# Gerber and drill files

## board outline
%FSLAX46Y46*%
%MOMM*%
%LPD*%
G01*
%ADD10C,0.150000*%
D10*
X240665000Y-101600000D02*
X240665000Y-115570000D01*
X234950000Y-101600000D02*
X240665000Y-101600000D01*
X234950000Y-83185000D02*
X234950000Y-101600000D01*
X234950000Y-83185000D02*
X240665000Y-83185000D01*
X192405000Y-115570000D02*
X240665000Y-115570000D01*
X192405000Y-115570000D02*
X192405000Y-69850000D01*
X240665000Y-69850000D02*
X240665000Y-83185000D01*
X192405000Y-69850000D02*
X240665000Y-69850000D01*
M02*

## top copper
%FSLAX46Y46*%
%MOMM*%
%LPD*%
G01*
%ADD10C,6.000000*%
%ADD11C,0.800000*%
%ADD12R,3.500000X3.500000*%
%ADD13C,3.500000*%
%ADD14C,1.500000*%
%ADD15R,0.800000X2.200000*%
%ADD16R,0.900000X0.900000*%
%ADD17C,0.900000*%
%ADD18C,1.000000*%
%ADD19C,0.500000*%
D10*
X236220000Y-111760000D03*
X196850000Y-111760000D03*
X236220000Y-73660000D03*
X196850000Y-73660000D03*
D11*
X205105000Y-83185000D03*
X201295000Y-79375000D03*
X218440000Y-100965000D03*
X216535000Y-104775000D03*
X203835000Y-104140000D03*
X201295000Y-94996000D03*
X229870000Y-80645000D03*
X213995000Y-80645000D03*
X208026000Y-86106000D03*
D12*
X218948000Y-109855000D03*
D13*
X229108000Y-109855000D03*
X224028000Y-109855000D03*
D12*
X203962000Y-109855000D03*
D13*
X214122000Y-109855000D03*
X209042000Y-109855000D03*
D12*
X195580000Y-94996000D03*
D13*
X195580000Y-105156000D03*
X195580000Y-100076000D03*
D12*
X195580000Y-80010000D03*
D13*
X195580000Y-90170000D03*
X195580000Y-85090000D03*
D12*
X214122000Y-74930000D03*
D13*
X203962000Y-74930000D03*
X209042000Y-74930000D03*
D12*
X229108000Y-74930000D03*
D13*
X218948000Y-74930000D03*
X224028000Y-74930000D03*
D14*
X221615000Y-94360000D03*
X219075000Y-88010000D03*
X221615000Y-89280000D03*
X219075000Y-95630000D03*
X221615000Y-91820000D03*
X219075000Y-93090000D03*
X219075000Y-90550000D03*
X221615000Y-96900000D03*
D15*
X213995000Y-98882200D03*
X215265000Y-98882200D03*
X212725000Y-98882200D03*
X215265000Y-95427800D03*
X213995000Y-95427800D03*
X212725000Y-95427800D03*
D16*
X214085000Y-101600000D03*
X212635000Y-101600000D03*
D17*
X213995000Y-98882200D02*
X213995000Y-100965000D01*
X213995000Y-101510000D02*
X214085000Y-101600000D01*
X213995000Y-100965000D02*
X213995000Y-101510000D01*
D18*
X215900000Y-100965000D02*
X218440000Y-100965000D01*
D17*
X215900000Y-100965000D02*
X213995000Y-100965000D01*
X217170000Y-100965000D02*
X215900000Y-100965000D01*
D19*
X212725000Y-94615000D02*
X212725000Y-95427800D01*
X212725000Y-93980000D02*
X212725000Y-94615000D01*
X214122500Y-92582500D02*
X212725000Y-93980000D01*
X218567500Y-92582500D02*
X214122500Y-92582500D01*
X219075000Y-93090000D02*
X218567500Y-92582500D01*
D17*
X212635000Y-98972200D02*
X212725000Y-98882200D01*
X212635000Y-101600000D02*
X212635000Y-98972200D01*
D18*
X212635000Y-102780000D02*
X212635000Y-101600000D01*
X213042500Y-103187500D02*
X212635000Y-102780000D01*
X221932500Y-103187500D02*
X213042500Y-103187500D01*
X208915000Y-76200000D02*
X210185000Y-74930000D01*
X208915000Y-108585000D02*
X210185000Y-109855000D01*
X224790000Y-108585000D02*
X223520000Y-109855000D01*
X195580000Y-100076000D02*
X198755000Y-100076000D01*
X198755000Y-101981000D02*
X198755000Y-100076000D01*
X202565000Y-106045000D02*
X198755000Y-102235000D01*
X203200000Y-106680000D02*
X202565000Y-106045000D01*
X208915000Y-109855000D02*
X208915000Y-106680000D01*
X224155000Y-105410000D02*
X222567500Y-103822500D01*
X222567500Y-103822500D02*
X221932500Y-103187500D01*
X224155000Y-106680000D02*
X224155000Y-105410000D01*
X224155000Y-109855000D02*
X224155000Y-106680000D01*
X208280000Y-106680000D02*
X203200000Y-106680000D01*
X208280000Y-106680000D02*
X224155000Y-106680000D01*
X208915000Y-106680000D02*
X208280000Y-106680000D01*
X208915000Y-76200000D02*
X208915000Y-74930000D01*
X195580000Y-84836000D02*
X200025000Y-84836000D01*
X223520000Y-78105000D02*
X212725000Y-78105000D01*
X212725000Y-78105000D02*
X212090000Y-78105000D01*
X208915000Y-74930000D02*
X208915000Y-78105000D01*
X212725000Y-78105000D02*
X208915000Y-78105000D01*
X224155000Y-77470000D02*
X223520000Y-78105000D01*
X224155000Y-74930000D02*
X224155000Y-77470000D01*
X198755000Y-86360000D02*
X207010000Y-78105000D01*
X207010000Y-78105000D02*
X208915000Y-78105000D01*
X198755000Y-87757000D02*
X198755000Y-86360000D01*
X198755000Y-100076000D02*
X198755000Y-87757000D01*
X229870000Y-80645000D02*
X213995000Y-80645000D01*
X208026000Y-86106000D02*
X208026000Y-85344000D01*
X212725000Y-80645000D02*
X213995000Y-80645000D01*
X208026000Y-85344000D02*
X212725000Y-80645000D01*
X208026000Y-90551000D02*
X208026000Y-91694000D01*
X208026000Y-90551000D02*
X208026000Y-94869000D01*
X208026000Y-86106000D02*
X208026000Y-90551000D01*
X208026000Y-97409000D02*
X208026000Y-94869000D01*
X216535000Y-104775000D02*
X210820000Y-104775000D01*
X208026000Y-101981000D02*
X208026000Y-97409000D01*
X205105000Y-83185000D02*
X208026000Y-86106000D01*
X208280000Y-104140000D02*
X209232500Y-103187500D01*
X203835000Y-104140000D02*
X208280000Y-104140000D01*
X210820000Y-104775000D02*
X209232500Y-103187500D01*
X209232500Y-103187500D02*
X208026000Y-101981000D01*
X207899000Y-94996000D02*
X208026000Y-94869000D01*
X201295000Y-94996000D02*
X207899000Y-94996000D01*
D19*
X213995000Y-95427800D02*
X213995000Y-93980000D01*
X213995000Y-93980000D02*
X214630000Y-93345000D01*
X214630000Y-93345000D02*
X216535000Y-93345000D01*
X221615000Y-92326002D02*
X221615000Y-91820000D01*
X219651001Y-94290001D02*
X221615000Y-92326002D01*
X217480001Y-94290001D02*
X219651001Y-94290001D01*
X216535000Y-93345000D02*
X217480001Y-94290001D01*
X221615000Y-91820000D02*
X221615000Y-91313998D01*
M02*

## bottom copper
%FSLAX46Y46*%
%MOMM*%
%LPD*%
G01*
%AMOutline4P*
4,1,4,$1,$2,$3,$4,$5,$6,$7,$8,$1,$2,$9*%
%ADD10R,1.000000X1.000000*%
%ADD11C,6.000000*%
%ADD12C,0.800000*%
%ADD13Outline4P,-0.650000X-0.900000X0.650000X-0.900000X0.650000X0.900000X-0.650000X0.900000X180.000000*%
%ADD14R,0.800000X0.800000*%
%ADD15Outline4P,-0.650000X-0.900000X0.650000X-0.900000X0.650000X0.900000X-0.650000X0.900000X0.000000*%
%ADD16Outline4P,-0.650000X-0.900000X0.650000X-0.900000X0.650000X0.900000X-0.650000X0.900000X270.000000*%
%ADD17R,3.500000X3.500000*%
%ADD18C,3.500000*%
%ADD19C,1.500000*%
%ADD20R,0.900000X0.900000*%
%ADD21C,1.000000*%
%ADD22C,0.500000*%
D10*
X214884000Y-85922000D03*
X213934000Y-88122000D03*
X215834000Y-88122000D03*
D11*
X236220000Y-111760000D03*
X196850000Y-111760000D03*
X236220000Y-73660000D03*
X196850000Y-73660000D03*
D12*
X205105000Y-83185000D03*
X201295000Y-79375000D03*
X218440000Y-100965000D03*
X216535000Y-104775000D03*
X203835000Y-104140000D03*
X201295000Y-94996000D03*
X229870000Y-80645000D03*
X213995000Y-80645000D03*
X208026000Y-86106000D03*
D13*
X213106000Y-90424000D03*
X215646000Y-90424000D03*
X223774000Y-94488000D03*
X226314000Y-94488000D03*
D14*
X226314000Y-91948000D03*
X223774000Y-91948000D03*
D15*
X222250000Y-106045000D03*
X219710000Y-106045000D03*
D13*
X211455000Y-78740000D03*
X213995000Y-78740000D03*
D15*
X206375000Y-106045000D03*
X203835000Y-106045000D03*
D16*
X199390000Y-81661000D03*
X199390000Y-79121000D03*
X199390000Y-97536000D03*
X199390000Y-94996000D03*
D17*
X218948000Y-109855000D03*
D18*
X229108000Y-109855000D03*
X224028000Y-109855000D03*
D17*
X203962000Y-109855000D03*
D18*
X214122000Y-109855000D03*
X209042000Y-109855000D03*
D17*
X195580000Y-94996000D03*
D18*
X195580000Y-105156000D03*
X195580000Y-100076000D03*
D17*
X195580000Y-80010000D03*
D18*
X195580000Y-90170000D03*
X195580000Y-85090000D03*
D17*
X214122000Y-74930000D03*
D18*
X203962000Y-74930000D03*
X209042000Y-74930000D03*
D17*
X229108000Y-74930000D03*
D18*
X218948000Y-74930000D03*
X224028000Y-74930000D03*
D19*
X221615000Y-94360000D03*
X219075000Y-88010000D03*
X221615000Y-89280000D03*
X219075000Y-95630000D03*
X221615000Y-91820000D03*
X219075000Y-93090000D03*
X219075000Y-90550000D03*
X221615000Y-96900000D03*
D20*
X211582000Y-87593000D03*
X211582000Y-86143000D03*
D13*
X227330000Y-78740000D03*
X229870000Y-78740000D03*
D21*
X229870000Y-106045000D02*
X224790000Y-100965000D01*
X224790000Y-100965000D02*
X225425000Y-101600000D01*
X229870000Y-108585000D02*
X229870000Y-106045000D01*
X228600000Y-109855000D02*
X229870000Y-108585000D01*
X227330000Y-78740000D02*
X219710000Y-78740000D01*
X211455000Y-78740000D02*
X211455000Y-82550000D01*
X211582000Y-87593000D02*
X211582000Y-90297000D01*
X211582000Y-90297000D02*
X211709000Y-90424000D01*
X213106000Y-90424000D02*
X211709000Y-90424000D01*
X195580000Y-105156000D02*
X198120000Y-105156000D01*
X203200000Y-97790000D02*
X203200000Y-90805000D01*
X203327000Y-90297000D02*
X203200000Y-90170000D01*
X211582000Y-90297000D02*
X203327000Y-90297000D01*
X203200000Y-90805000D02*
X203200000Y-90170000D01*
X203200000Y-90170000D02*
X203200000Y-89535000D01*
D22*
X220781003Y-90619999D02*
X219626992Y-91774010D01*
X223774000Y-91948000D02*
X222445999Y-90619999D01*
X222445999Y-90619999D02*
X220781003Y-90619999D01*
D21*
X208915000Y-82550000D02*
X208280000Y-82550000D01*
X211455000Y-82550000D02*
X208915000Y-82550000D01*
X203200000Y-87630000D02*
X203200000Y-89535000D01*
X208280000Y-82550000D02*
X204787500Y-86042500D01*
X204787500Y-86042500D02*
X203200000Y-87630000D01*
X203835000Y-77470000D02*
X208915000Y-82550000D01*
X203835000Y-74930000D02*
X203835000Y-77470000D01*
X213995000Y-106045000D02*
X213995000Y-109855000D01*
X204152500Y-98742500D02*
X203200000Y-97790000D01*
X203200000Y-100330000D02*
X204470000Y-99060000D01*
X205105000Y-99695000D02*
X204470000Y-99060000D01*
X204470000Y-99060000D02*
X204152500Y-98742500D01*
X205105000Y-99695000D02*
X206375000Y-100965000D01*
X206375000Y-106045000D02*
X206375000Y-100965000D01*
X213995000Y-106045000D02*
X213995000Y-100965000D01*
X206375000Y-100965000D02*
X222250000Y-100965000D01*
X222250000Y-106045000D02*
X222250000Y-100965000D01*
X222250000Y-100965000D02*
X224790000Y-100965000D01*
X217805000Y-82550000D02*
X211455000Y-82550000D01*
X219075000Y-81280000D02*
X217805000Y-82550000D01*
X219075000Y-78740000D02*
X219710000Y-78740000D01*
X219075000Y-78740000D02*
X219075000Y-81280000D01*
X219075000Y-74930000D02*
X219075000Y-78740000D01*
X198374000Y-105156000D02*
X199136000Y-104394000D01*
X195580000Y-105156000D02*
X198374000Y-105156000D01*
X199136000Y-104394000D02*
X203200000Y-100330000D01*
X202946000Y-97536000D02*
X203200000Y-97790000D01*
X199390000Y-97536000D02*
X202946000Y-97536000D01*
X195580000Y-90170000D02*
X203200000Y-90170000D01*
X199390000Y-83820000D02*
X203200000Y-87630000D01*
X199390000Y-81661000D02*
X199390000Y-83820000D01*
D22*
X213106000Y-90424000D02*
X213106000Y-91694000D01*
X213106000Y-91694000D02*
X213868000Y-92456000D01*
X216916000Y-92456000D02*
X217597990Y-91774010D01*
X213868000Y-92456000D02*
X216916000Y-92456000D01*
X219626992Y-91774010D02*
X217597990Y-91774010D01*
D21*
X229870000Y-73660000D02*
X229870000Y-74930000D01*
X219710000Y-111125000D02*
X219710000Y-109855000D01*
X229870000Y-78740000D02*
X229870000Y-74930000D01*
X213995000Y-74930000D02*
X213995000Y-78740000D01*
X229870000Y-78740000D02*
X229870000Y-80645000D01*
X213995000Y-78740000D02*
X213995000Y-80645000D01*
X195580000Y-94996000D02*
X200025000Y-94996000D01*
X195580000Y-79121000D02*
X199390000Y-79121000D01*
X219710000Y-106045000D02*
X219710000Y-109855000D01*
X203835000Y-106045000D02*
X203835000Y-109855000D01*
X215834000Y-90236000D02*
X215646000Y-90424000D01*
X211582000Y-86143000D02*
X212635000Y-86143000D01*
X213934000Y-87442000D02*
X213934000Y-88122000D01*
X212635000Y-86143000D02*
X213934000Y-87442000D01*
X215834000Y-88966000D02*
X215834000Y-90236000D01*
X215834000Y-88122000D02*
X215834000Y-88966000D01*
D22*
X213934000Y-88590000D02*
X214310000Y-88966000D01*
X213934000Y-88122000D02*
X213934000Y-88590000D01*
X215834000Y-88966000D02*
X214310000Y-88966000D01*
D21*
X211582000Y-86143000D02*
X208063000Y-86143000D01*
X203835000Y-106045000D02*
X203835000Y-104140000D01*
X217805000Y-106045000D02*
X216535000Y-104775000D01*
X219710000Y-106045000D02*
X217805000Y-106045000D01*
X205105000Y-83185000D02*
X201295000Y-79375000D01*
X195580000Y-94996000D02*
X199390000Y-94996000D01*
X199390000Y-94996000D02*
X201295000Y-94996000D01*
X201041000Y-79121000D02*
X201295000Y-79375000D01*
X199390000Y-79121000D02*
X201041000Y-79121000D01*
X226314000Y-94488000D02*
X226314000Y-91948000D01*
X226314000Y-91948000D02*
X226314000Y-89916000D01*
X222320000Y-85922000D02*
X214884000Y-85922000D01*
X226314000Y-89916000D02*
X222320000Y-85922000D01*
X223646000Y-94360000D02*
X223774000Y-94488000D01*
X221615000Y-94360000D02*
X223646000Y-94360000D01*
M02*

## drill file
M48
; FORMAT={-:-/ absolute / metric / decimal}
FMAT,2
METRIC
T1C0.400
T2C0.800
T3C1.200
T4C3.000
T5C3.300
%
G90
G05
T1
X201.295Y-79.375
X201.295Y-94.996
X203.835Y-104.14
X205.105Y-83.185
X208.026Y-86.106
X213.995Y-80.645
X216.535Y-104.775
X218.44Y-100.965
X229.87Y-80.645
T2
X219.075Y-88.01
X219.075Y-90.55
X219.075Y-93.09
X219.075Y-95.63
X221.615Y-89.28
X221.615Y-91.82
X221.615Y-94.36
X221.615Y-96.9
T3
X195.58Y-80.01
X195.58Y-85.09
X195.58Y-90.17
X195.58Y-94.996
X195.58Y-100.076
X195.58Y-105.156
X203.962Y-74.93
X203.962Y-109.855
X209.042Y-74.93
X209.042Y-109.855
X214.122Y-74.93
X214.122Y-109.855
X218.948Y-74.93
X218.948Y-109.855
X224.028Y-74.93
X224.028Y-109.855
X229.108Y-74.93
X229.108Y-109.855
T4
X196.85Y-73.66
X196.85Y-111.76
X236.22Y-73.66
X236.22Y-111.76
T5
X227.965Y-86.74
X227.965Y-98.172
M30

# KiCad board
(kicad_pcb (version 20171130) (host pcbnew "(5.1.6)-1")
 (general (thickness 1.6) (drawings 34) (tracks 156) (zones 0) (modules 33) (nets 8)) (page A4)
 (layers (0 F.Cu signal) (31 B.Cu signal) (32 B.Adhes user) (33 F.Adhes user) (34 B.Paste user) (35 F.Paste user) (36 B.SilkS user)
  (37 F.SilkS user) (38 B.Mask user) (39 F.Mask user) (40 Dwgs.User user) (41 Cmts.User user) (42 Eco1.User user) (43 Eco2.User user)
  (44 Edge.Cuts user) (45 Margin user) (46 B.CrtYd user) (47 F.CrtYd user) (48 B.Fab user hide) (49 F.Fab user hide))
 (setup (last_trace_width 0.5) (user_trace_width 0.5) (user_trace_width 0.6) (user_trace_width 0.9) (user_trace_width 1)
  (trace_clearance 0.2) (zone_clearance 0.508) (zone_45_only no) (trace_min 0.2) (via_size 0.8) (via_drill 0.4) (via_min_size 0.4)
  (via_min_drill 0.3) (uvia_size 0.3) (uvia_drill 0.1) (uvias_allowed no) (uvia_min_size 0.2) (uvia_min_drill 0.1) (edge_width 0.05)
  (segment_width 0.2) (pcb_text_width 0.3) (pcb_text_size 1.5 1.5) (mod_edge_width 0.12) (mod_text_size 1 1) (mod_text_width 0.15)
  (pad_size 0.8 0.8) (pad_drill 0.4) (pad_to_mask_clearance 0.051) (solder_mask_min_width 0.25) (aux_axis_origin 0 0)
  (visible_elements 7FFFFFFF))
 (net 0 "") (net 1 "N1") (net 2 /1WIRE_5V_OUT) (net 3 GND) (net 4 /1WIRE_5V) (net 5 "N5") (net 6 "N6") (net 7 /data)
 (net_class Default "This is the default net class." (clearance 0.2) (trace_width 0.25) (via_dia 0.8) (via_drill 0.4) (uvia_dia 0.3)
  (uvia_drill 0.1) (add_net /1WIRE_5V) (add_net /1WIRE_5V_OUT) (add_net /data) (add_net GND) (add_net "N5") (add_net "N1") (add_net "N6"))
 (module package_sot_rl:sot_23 (layer B.Cu) (at 214.884 87.122 90)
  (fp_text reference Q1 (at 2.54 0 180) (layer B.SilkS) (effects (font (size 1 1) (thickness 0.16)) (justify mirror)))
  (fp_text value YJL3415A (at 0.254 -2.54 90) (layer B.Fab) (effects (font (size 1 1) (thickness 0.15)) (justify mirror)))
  (pad 3 smd rect (at 1.2 0 90) (size 1 1) (layers B.Cu B.Paste B.Mask) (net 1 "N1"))
  (pad 2 smd rect (at -1 -0.95 90) (size 1 1) (layers B.Cu B.Paste B.Mask) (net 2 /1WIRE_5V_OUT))
  (pad 1 smd rect (at -1 0.95 90) (size 1 1) (layers B.Cu B.Paste B.Mask) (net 2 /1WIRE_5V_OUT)))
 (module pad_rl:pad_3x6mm (layer F.Cu) (at 236.22 111.76)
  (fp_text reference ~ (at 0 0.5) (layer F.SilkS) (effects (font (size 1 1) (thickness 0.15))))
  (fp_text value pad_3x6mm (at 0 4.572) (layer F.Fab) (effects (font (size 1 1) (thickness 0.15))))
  (pad ~ thru_hole circle (at 0 0) (size 6 6) (drill 3) (layers *.Cu *.Mask)))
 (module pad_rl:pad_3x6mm (layer F.Cu) (at 196.85 111.76)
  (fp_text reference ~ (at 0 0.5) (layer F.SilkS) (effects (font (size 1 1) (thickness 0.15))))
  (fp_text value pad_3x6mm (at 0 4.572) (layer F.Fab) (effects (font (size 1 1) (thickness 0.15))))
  (pad ~ thru_hole circle (at 0 0) (size 6 6) (drill 3) (layers *.Cu *.Mask)))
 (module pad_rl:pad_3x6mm (layer F.Cu) (at 236.22 73.66)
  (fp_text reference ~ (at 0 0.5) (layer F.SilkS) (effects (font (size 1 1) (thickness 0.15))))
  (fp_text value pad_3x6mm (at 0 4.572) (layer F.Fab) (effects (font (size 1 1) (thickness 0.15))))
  (pad ~ thru_hole circle (at 0 0) (size 6 6) (drill 3) (layers *.Cu *.Mask)))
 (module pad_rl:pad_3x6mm (layer F.Cu) (at 196.85 73.66)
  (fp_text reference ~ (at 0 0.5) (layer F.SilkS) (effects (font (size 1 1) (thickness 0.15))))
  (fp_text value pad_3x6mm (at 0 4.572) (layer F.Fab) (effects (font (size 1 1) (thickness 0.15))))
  (pad ~ thru_hole circle (at 0 0) (size 6 6) (drill 3) (layers *.Cu *.Mask)))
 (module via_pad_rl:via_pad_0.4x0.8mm (layer F.Cu) (at 205.105 83.185 90)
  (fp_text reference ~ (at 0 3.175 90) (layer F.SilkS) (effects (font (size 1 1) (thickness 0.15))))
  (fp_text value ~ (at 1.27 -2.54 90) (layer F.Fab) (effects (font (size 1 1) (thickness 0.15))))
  (pad ~ thru_hole circle (at 0 0 90) (size 0.8 0.8) (drill 0.4) (layers *.Cu *.Mask) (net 2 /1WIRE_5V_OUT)))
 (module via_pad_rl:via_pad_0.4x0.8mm (layer F.Cu) (at 201.295 79.375 90)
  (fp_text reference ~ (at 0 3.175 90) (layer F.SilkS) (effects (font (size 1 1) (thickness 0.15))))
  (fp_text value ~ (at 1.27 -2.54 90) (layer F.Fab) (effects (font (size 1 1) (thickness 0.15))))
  (pad ~ thru_hole circle (at 0 0 90) (size 0.8 0.8) (drill 0.4) (layers *.Cu *.Mask) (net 2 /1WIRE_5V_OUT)))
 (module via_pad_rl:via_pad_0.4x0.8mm (layer F.Cu) (at 218.44 100.965 90)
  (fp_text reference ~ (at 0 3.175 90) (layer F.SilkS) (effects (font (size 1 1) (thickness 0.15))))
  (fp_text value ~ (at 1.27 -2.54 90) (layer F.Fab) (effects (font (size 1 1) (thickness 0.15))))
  (pad ~ thru_hole circle (at 0 0 90) (size 0.8 0.8) (drill 0.4) (layers *.Cu *.Mask) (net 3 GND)))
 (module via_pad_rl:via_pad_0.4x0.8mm (layer F.Cu) (at 216.535 104.775 90)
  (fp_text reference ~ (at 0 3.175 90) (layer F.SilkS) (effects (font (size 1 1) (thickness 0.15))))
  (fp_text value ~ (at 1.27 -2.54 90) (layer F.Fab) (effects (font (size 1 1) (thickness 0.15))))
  (pad ~ thru_hole circle (at 0 0 90) (size 0.8 0.8) (drill 0.4) (layers *.Cu *.Mask) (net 2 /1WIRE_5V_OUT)))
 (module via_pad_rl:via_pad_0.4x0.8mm (layer F.Cu) (at 203.835 104.14 90)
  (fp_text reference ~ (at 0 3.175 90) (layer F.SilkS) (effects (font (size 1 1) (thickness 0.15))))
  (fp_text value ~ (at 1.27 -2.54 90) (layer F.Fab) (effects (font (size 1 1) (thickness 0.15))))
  (pad ~ thru_hole circle (at 0 0 90) (size 0.8 0.8) (drill 0.4) (layers *.Cu *.Mask) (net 2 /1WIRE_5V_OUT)))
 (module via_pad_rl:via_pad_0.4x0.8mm (layer F.Cu) (at 201.295 94.996 90)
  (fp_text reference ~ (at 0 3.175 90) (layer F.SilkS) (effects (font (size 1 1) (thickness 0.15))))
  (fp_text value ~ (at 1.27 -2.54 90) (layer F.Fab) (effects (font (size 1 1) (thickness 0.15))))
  (pad ~ thru_hole circle (at 0 0 90) (size 0.8 0.8) (drill 0.4) (layers *.Cu *.Mask) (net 2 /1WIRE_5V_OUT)))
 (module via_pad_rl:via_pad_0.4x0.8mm (layer F.Cu) (at 229.87 80.645 90)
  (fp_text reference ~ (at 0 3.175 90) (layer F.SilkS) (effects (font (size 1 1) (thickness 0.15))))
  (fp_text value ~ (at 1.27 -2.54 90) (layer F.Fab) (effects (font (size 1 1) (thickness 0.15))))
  (pad ~ thru_hole circle (at 0 0 90) (size 0.8 0.8) (drill 0.4) (layers *.Cu *.Mask) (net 2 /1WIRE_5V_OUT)))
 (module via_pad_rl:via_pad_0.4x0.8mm (layer F.Cu) (at 213.995 80.645 90)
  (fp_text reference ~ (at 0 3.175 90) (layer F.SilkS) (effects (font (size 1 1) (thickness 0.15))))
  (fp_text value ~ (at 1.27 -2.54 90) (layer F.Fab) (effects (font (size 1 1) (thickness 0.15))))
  (pad ~ thru_hole circle (at 0 0 90) (size 0.8 0.8) (drill 0.4) (layers *.Cu *.Mask) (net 2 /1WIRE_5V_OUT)))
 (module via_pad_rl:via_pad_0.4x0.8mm (layer F.Cu) (at 208.026 86.106 90)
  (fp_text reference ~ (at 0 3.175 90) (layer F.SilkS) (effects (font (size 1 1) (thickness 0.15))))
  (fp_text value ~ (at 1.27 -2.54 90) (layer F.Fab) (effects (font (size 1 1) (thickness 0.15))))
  (pad ~ thru_hole circle (at 0 0 90) (size 0.8 0.8) (drill 0.4) (layers *.Cu *.Mask) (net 2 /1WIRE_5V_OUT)))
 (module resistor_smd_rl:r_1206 (layer B.Cu) (at 214.376 90.424 180)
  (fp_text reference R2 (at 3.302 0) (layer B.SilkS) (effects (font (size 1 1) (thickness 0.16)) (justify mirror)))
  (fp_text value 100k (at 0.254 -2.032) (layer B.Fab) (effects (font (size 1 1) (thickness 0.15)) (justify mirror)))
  (pad 2 smd trapezoid (at 1.27 0 180) (size 1.3 1.8) (layers B.Cu B.Paste B.Mask) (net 3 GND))
  (pad 1 smd trapezoid (at -1.27 0 180) (size 1.3 1.8) (layers B.Cu B.Paste B.Mask) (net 2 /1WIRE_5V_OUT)))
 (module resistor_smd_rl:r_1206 (layer B.Cu) (at 225.044 94.488 180)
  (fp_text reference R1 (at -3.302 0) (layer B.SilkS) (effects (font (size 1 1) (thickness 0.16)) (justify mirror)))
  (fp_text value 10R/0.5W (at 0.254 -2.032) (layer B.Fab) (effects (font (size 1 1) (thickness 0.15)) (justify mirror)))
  (pad 2 smd trapezoid (at 1.27 0 180) (size 1.3 1.8) (layers B.Cu B.Paste B.Mask) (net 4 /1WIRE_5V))
  (pad 1 smd trapezoid (at -1.27 0 180) (size 1.3 1.8) (layers B.Cu B.Paste B.Mask) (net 1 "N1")))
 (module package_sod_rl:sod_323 (layer B.Cu) (at 225.044 91.948 180)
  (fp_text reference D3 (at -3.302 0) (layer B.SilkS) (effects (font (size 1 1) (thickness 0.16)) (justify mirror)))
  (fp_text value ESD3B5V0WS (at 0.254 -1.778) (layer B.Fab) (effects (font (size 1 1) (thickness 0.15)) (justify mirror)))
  (pad 1 smd rect (at -1.27 0 180) (size 0.8 0.8) (layers B.Cu B.Paste B.Mask) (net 1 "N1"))
  (pad 2 smd rect (at 1.27 0 180) (size 0.8 0.8) (layers B.Cu B.Paste B.Mask) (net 3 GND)))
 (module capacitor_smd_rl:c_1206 (layer B.Cu) (at 220.98 106.045)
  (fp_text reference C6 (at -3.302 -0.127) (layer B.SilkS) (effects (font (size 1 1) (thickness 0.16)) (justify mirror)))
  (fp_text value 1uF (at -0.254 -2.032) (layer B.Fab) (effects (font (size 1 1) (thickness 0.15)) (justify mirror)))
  (pad 2 smd trapezoid (at 1.27 0) (size 1.3 1.8) (layers B.Cu B.Paste B.Mask) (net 3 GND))
  (pad 1 smd trapezoid (at -1.27 0) (size 1.3 1.8) (layers B.Cu B.Paste B.Mask) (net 2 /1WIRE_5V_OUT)))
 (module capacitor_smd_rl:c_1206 (layer B.Cu) (at 212.725 78.74 180)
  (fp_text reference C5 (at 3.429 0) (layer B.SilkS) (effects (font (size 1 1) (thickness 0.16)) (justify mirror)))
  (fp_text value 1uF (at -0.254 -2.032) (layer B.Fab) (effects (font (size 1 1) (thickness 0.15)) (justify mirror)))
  (pad 2 smd trapezoid (at 1.27 0 180) (size 1.3 1.8) (layers B.Cu B.Paste B.Mask) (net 3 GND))
  (pad 1 smd trapezoid (at -1.27 0 180) (size 1.3 1.8) (layers B.Cu B.Paste B.Mask) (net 2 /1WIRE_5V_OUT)))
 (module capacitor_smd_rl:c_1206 (layer B.Cu) (at 205.105 106.045)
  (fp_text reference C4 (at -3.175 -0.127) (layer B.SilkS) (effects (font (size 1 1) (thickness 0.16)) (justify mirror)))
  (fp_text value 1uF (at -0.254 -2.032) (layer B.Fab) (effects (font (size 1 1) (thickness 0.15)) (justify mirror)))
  (pad 2 smd trapezoid (at 1.27 0) (size 1.3 1.8) (layers B.Cu B.Paste B.Mask) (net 3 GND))
  (pad 1 smd trapezoid (at -1.27 0) (size 1.3 1.8) (layers B.Cu B.Paste B.Mask) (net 2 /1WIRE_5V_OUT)))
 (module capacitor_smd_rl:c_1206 (layer B.Cu) (at 199.39 80.391 270)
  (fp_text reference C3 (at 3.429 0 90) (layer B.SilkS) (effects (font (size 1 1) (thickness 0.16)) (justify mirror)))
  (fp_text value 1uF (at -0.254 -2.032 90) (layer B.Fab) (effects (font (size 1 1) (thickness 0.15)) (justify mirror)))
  (pad 2 smd trapezoid (at 1.27 0 270) (size 1.3 1.8) (layers B.Cu B.Paste B.Mask) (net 3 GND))
  (pad 1 smd trapezoid (at -1.27 0 270) (size 1.3 1.8) (layers B.Cu B.Paste B.Mask) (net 2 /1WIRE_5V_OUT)))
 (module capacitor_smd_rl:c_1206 (layer B.Cu) (at 199.39 96.266 270)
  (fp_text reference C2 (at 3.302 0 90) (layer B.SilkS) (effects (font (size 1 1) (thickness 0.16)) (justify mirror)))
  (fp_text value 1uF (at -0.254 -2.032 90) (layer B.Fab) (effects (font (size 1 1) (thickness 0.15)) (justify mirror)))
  (pad 2 smd trapezoid (at 1.27 0 270) (size 1.3 1.8) (layers B.Cu B.Paste B.Mask) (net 3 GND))
  (pad 1 smd trapezoid (at -1.27 0 270) (size 1.3 1.8) (layers B.Cu B.Paste B.Mask) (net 2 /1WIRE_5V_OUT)))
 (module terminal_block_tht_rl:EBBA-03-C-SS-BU (layer F.Cu) (at 224.028 109.855)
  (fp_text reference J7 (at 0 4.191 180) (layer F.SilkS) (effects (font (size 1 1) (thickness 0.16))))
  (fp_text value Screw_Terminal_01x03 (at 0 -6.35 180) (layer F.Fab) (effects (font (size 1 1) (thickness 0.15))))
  (pad 1 thru_hole rect (at -5.08 0 180) (size 3.5 3.5) (drill 1.2) (layers *.Cu *.Mask) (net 2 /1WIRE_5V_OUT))
  (pad 3 thru_hole circle (at 5.08 0 180) (size 3.5 3.5) (drill 1.2) (layers *.Cu *.Mask) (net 3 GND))
  (pad 2 thru_hole circle (at 0 0 180) (size 3.5 3.5) (drill 1.2) (layers *.Cu *.Mask) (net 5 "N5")))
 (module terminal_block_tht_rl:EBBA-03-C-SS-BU (layer F.Cu) (at 209.042 109.855)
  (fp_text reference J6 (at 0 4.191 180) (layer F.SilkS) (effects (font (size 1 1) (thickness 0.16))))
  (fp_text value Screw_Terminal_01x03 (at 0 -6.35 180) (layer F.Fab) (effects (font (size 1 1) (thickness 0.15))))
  (pad 1 thru_hole rect (at -5.08 0 180) (size 3.5 3.5) (drill 1.2) (layers *.Cu *.Mask) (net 2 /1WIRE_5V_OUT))
  (pad 3 thru_hole circle (at 5.08 0 180) (size 3.5 3.5) (drill 1.2) (layers *.Cu *.Mask) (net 3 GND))
  (pad 2 thru_hole circle (at 0 0 180) (size 3.5 3.5) (drill 1.2) (layers *.Cu *.Mask) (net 5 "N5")))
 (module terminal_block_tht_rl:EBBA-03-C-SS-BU (layer F.Cu) (at 195.58 100.076 270)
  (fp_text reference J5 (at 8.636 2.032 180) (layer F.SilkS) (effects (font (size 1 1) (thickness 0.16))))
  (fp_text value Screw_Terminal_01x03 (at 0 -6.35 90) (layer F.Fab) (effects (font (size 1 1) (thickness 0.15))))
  (pad 1 thru_hole rect (at -5.08 0 90) (size 3.5 3.5) (drill 1.2) (layers *.Cu *.Mask) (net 2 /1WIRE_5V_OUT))
  (pad 3 thru_hole circle (at 5.08 0 90) (size 3.5 3.5) (drill 1.2) (layers *.Cu *.Mask) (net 3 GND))
  (pad 2 thru_hole circle (at 0 0 90) (size 3.5 3.5) (drill 1.2) (layers *.Cu *.Mask) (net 5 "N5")))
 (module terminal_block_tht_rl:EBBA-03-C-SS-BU (layer F.Cu) (at 195.58 85.09 270)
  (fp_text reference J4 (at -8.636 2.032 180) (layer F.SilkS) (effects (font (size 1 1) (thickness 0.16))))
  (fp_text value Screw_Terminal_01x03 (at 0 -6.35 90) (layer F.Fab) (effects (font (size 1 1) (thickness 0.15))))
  (pad 1 thru_hole rect (at -5.08 0 90) (size 3.5 3.5) (drill 1.2) (layers *.Cu *.Mask) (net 2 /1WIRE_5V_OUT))
  (pad 3 thru_hole circle (at 5.08 0 90) (size 3.5 3.5) (drill 1.2) (layers *.Cu *.Mask) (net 3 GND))
  (pad 2 thru_hole circle (at 0 0 90) (size 3.5 3.5) (drill 1.2) (layers *.Cu *.Mask) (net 5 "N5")))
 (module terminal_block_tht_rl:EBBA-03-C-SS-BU (layer F.Cu) (at 209.042 74.93 180)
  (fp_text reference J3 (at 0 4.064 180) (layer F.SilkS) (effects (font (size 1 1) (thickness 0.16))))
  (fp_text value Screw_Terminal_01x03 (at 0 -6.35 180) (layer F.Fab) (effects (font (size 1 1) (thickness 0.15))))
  (pad 1 thru_hole rect (at -5.08 0) (size 3.5 3.5) (drill 1.2) (layers *.Cu *.Mask) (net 2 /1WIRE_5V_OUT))
  (pad 3 thru_hole circle (at 5.08 0) (size 3.5 3.5) (drill 1.2) (layers *.Cu *.Mask) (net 3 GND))
  (pad 2 thru_hole circle (at 0 0) (size 3.5 3.5) (drill 1.2) (layers *.Cu *.Mask) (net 5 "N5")))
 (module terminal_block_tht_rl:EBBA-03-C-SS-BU (layer F.Cu) (at 224.028 74.93 180)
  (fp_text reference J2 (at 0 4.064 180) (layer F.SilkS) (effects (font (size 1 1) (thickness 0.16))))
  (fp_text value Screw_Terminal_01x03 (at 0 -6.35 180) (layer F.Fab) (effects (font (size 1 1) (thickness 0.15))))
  (pad 1 thru_hole rect (at -5.08 0) (size 3.5 3.5) (drill 1.2) (layers *.Cu *.Mask) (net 2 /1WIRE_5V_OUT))
  (pad 3 thru_hole circle (at 5.08 0) (size 3.5 3.5) (drill 1.2) (layers *.Cu *.Mask) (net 3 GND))
  (pad 2 thru_hole circle (at 0 0) (size 3.5 3.5) (drill 1.2) (layers *.Cu *.Mask) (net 5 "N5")))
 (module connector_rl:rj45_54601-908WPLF (layer F.Cu) (at 227.965 92.456 90)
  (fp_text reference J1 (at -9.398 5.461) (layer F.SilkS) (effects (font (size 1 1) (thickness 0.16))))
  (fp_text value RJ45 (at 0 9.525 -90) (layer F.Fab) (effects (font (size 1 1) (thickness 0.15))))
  (pad 3 thru_hole circle (at -1.904 -6.35 90) (size 1.5 1.5) (drill 0.8) (layers *.Cu *.Mask) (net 4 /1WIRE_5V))
  (pad 8 thru_hole circle (at 4.446 -8.89 90) (size 1.5 1.5) (drill 0.8) (layers *.Cu *.Mask))
  (pad "" np_thru_hole circle (at -5.716 0 90) (size 3.3 3.3) (drill 3.3) (layers *.Cu *.SilkS *.Mask))
  (pad 7 thru_hole circle (at 3.176 -6.35 90) (size 1.5 1.5) (drill 0.8) (layers *.Cu *.Mask))
  (pad 2 thru_hole circle (at -3.174 -8.89 90) (size 1.5 1.5) (drill 0.8) (layers *.Cu *.Mask))
  (pad 5 thru_hole circle (at 0.636 -6.35 90) (size 1.5 1.5) (drill 0.8) (layers *.Cu *.Mask) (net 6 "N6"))
  (pad 4 thru_hole circle (at -0.634 -8.89 90) (size 1.5 1.5) (drill 0.8) (layers *.Cu *.Mask) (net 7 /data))
  (pad 6 thru_hole circle (at 1.906 -8.89 270) (size 1.5 1.5) (drill 0.8) (layers *.Cu *.Mask))
  (pad 1 thru_hole circle (at -4.444 -6.35 90) (size 1.5 1.5) (drill 0.8) (layers *.Cu *.Mask))
  (pad "" np_thru_hole circle (at 5.716 0 90) (size 3.3 3.3) (drill 3.3) (layers *.Cu *.SilkS *.Mask)))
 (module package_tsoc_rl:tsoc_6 (layer F.Cu) (at 213.995 97.155 90)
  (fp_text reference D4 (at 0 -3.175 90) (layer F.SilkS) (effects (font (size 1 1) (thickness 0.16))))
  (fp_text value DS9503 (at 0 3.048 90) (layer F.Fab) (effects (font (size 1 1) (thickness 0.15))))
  (pad 2 smd rect (at -1.7272 0 90) (size 2.2 0.8) (layers F.Cu F.Paste F.Mask) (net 3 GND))
  (pad 3 smd rect (at -1.7272 1.27 90) (size 2.2 0.8) (layers F.Cu F.Paste F.Mask))
  (pad 1 smd rect (at -1.7272 -1.27 90) (size 2.2 0.8) (layers F.Cu F.Paste F.Mask) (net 5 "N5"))
  (pad 4 smd rect (at 1.7272 1.27 90) (size 2.2 0.8) (layers F.Cu F.Paste F.Mask))
  (pad 5 smd rect (at 1.7272 0 90) (size 2.2 0.8) (layers F.Cu F.Paste F.Mask) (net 6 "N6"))
  (pad 6 smd rect (at 1.7272 -1.27 90) (size 2.2 0.8) (layers F.Cu F.Paste F.Mask) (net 7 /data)))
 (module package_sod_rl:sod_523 (layer F.Cu) (at 213.36 101.6)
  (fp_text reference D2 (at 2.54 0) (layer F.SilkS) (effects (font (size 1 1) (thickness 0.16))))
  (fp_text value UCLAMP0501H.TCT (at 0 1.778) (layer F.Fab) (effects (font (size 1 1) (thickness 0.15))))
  (pad 2 smd rect (at 0.725 0) (size 0.9 0.9) (layers F.Cu F.Paste F.Mask) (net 3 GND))
  (pad 1 smd rect (at -0.725 0) (size 0.9 0.9) (layers F.Cu F.Paste F.Mask) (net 5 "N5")))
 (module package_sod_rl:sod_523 (layer B.Cu) (at 211.582 86.868 270)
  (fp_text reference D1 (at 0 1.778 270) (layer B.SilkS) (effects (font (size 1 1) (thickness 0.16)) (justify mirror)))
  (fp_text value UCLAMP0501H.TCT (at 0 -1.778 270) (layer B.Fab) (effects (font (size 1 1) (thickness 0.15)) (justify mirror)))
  (pad 2 smd rect (at 0.725 0 270) (size 0.9 0.9) (layers B.Cu B.Paste B.Mask) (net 3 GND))
  (pad 1 smd rect (at -0.725 0 270) (size 0.9 0.9) (layers B.Cu B.Paste B.Mask) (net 2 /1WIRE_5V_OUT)))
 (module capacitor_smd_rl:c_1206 (layer B.Cu) (at 228.6 78.74 180)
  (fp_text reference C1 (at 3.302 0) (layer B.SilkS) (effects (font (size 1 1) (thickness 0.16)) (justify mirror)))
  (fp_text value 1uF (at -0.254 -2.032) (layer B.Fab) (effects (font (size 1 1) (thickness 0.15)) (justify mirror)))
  (pad 2 smd trapezoid (at 1.27 0 180) (size 1.3 1.8) (layers B.Cu B.Paste B.Mask) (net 3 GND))
  (pad 1 smd trapezoid (at -1.27 0 180) (size 1.3 1.8) (layers B.Cu B.Paste B.Mask) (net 2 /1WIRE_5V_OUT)))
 (gr_line (start 240.665 101.6) (end 240.665 115.57) (layer Edge.Cuts) (width 0.15))
 (gr_line (start 234.95 101.6) (end 240.665 101.6) (layer Edge.Cuts) (width 0.15))
 (gr_line (start 234.95 83.185) (end 234.95 101.6) (layer Edge.Cuts) (width 0.15))
 (gr_line (start 234.95 83.185) (end 240.665 83.185) (layer Edge.Cuts) (width 0.15))
 (gr_line (start 192.405 115.57) (end 240.665 115.57) (layer Edge.Cuts) (width 0.15))
 (gr_line (start 192.405 115.57) (end 192.405 69.85) (layer Edge.Cuts) (width 0.15))
 (gr_line (start 240.665 69.85) (end 240.665 83.185) (layer Edge.Cuts) (width 0.15))
 (gr_line (start 192.405 69.85) (end 240.665 69.85) (layer Edge.Cuts) (width 0.15))
 (segment (start 229.87 106.045) (end 224.79 100.965) (width 1) (layer B.Cu) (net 3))
 (segment (start 224.79 100.965) (end 225.425 101.6) (width 1) (layer B.Cu) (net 3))
 (segment (start 229.87 108.585) (end 229.87 106.045) (width 1) (layer B.Cu) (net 3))
 (segment (start 228.6 109.855) (end 229.87 108.585) (width 1) (layer B.Cu) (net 3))
 (segment (start 213.995 98.8822) (end 213.995 100.965) (width 0.9) (layer F.Cu) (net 3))
 (segment (start 213.995 101.51) (end 214.085 101.6) (width 0.9) (layer F.Cu) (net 3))
 (segment (start 213.995 100.965) (end 213.995 101.51) (width 0.9) (layer F.Cu) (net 3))
 (segment (start 227.33 78.74) (end 219.71 78.74) (width 1) (layer B.Cu) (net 3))
 (segment (start 211.455 78.74) (end 211.455 82.55) (width 1) (layer B.Cu) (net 3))
 (segment (start 211.582 87.593) (end 211.582 90.297) (width 1) (layer B.Cu) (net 3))
 (segment (start 211.582 90.297) (end 211.709 90.424) (width 1) (layer B.Cu) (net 3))
 (segment (start 213.106 90.424) (end 211.709 90.424) (width 1) (layer B.Cu) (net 3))
 (segment (start 195.58 105.156) (end 198.12 105.156) (width 1) (layer B.Cu) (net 3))
 (segment (start 203.2 97.79) (end 203.2 90.805) (width 1) (layer B.Cu) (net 3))
 (segment (start 203.327 90.297) (end 203.2 90.17) (width 1) (layer B.Cu) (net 3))
 (segment (start 211.582 90.297) (end 203.327 90.297) (width 1) (layer B.Cu) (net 3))
 (segment (start 203.2 90.805) (end 203.2 90.17) (width 1) (layer B.Cu) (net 3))
 (segment (start 203.2 90.17) (end 203.2 89.535) (width 1) (layer B.Cu) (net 3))
 (segment (start 220.781003 90.619999) (end 219.626992 91.77401) (width 0.5) (layer B.Cu) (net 3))
 (segment (start 223.774 91.948) (end 222.445999 90.619999) (width 0.5) (layer B.Cu) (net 3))
 (segment (start 222.445999 90.619999) (end 220.781003 90.619999) (width 0.5) (layer B.Cu) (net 3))
 (segment (start 208.915 82.55) (end 208.28 82.55) (width 1) (layer B.Cu) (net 3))
 (segment (start 211.455 82.55) (end 208.915 82.55) (width 1) (layer B.Cu) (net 3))
 (segment (start 203.2 87.63) (end 203.2 89.535) (width 1) (layer B.Cu) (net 3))
 (segment (start 208.28 82.55) (end 204.7875 86.0425) (width 1) (layer B.Cu) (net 3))
 (segment (start 204.7875 86.0425) (end 203.2 87.63) (width 1) (layer B.Cu) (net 3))
 (segment (start 203.835 77.47) (end 208.915 82.55) (width 1) (layer B.Cu) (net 3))
 (segment (start 203.835 74.93) (end 203.835 77.47) (width 1) (layer B.Cu) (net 3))
 (segment (start 213.995 106.045) (end 213.995 109.855) (width 1) (layer B.Cu) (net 3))
 (segment (start 204.1525 98.7425) (end 203.2 97.79) (width 1) (layer B.Cu) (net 3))
 (segment (start 203.2 100.33) (end 204.47 99.06) (width 1) (layer B.Cu) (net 3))
 (segment (start 205.105 99.695) (end 204.47 99.06) (width 1) (layer B.Cu) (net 3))
 (segment (start 204.47 99.06) (end 204.1525 98.7425) (width 1) (layer B.Cu) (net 3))
 (segment (start 205.105 99.695) (end 206.375 100.965) (width 1) (layer B.Cu) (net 3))
 (segment (start 206.375 106.045) (end 206.375 100.965) (width 1) (layer B.Cu) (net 3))
 (segment (start 215.9 100.965) (end 218.44 100.965) (width 1) (layer F.Cu) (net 3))
 (segment (start 215.9 100.965) (end 213.995 100.965) (width 0.9) (layer F.Cu) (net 3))
 (segment (start 217.17 100.965) (end 215.9 100.965) (width 0.9) (layer F.Cu) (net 3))
 (segment (start 213.995 106.045) (end 213.995 100.965) (width 1) (layer B.Cu) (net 3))
 (segment (start 206.375 100.965) (end 222.25 100.965) (width 1) (layer B.Cu) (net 3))
 (segment (start 222.25 106.045) (end 222.25 100.965) (width 1) (layer B.Cu) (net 3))
 (segment (start 222.25 100.965) (end 224.79 100.965) (width 1) (layer B.Cu) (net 3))
 (segment (start 217.805 82.55) (end 211.455 82.55) (width 1) (layer B.Cu) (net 3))
 (segment (start 219.075 81.28) (end 217.805 82.55) (width 1) (layer B.Cu) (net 3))
 (segment (start 219.075 78.74) (end 219.71 78.74) (width 1) (layer B.Cu) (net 3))
 (segment (start 219.075 78.74) (end 219.075 81.28) (width 1) (layer B.Cu) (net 3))
 (segment (start 219.075 74.93) (end 219.075 78.74) (width 1) (layer B.Cu) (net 3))
 (segment (start 198.374 105.156) (end 199.136 104.394) (width 1) (layer B.Cu) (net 3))
 (segment (start 195.58 105.156) (end 198.374 105.156) (width 1) (layer B.Cu) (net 3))
 (segment (start 199.136 104.394) (end 203.2 100.33) (width 1) (layer B.Cu) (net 3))
 (segment (start 202.946 97.536) (end 203.2 97.79) (width 1) (layer B.Cu) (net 3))
 (segment (start 199.39 97.536) (end 202.946 97.536) (width 1) (layer B.Cu) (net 3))
 (segment (start 195.58 90.17) (end 203.2 90.17) (width 1) (layer B.Cu) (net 3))
 (segment (start 199.39 83.82) (end 203.2 87.63) (width 1) (layer B.Cu) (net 3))
 (segment (start 199.39 81.661) (end 199.39 83.82) (width 1) (layer B.Cu) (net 3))
 (segment (start 213.106 90.424) (end 213.106 91.694) (width 0.5) (layer B.Cu) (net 3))
 (segment (start 213.106 91.694) (end 213.868 92.456) (width 0.5) (layer B.Cu) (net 3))
 (segment (start 216.916 92.456) (end 217.59799 91.77401) (width 0.5) (layer B.Cu) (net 3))
 (segment (start 213.868 92.456) (end 216.916 92.456) (width 0.5) (layer B.Cu) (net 3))
 (segment (start 219.626992 91.77401) (end 217.59799 91.77401) (width 0.5) (layer B.Cu) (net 3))
 (segment (start 212.725 94.615) (end 212.725 95.4278) (width 0.5) (layer F.Cu) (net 7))
 (segment (start 212.725 93.98) (end 212.725 94.615) (width 0.5) (layer F.Cu) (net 7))
 (segment (start 214.1225 92.5825) (end 212.725 93.98) (width 0.5) (layer F.Cu) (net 7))
 (segment (start 218.5675 92.5825) (end 214.1225 92.5825) (width 0.5) (layer F.Cu) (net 7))
 (segment (start 219.075 93.09) (end 218.5675 92.5825) (width 0.5) (layer F.Cu) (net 7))
 (segment (start 212.635 98.9722) (end 212.725 98.8822) (width 0.9) (layer F.Cu) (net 5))
 (segment (start 212.635 101.6) (end 212.635 98.9722) (width 0.9) (layer F.Cu) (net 5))
 (segment (start 212.635 102.78) (end 212.635 101.6) (width 1) (layer F.Cu) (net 5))
 (segment (start 213.0425 103.1875) (end 212.635 102.78) (width 1) (layer F.Cu) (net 5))
 (segment (start 221.9325 103.1875) (end 213.0425 103.1875) (width 1) (layer F.Cu) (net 5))
 (segment (start 208.915 76.2) (end 210.185 74.93) (width 1) (layer F.Cu) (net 5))
 (segment (start 208.915 108.585) (end 210.185 109.855) (width 1) (layer F.Cu) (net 5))
 (segment (start 224.79 108.585) (end 223.52 109.855) (width 1) (layer F.Cu) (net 5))
 (segment (start 195.58 100.076) (end 198.755 100.076) (width 1) (layer F.Cu) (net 5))
 (segment (start 198.755 101.981) (end 198.755 100.076) (width 1) (layer F.Cu) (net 5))
 (segment (start 202.565 106.045) (end 198.755 102.235) (width 1) (layer F.Cu) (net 5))
 (segment (start 203.2 106.68) (end 202.565 106.045) (width 1) (layer F.Cu) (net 5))
 (segment (start 208.915 109.855) (end 208.915 106.68) (width 1) (layer F.Cu) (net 5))
 (segment (start 224.155 105.41) (end 222.5675 103.8225) (width 1) (layer F.Cu) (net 5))
 (segment (start 222.5675 103.8225) (end 221.9325 103.1875) (width 1) (layer F.Cu) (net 5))
 (segment (start 224.155 106.68) (end 224.155 105.41) (width 1) (layer F.Cu) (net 5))
 (segment (start 224.155 109.855) (end 224.155 106.68) (width 1) (layer F.Cu) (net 5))
 (segment (start 208.28 106.68) (end 203.2 106.68) (width 1) (layer F.Cu) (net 5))
 (segment (start 208.28 106.68) (end 224.155 106.68) (width 1) (layer F.Cu) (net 5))
 (segment (start 208.915 106.68) (end 208.28 106.68) (width 1) (layer F.Cu) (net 5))
 (segment (start 208.915 76.2) (end 208.915 74.93) (width 1) (layer F.Cu) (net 5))
 (segment (start 195.58 84.836) (end 200.025 84.836) (width 1) (layer F.Cu) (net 5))
 (segment (start 223.52 78.105) (end 212.725 78.105) (width 1) (layer F.Cu) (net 5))
 (segment (start 212.725 78.105) (end 212.09 78.105) (width 1) (layer F.Cu) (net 5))
 (segment (start 208.915 74.93) (end 208.915 78.105) (width 1) (layer F.Cu) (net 5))
 (segment (start 212.725 78.105) (end 208.915 78.105) (width 1) (layer F.Cu) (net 5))
 (segment (start 224.155 77.47) (end 223.52 78.105) (width 1) (layer F.Cu) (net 5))
 (segment (start 224.155 74.93) (end 224.155 77.47) (width 1) (layer F.Cu) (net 5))
 (segment (start 198.755 86.36) (end 207.01 78.105) (width 1) (layer F.Cu) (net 5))
 (segment (start 207.01 78.105) (end 208.915 78.105) (width 1) (layer F.Cu) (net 5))
 (segment (start 198.755 87.757) (end 198.755 86.36) (width 1) (layer F.Cu) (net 5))
 (segment (start 198.755 100.076) (end 198.755 87.757) (width 1) (layer F.Cu) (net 5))
 (segment (start 229.87 73.66) (end 229.87 74.93) (width 1) (layer B.Cu) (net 2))
 (segment (start 219.71 111.125) (end 219.71 109.855) (width 1) (layer B.Cu) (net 2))
 (segment (start 229.87 78.74) (end 229.87 74.93) (width 1) (layer B.Cu) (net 2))
 (segment (start 213.995 74.93) (end 213.995 78.74) (width 1) (layer B.Cu) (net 2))
 (segment (start 229.87 78.74) (end 229.87 80.645) (width 1) (layer B.Cu) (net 2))
 (segment (start 213.995 78.74) (end 213.995 80.645) (width 1) (layer B.Cu) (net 2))
 (segment (start 229.87 80.645) (end 213.995 80.645) (width 1) (layer F.Cu) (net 2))
 (segment (start 195.58 94.996) (end 200.025 94.996) (width 1) (layer B.Cu) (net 2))
 (segment (start 195.58 79.121) (end 199.39 79.121) (width 1) (layer B.Cu) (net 2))
 (segment (start 219.71 106.045) (end 219.71 109.855) (width 1) (layer B.Cu) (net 2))
 (segment (start 203.835 106.045) (end 203.835 109.855) (width 1) (layer B.Cu) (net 2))
 (segment (start 215.834 90.236) (end 215.646 90.424) (width 1) (layer B.Cu) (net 2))
 (segment (start 211.582 86.143) (end 212.635 86.143) (width 1) (layer B.Cu) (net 2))
 (segment (start 213.934 87.442) (end 213.934 88.122) (width 1) (layer B.Cu) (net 2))
 (segment (start 212.635 86.143) (end 213.934 87.442) (width 1) (layer B.Cu) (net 2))
 (segment (start 215.834 88.966) (end 215.834 90.236) (width 1) (layer B.Cu) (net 2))
 (segment (start 215.834 88.122) (end 215.834 88.966) (width 1) (layer B.Cu) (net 2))
 (segment (start 213.934 88.59) (end 214.31 88.966) (width 0.5) (layer B.Cu) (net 2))
 (segment (start 213.934 88.122) (end 213.934 88.59) (width 0.5) (layer B.Cu) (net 2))
 (segment (start 215.834 88.966) (end 214.31 88.966) (width 0.5) (layer B.Cu) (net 2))
 (segment (start 211.582 86.143) (end 208.063 86.143) (width 1) (layer B.Cu) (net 2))
 (segment (start 208.026 86.106) (end 208.026 85.344) (width 1) (layer F.Cu) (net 2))
 (segment (start 212.725 80.645) (end 213.995 80.645) (width 1) (layer F.Cu) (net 2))
 (segment (start 208.026 85.344) (end 212.725 80.645) (width 1) (layer F.Cu) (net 2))
 (segment (start 203.835 106.045) (end 203.835 104.14) (width 1) (layer B.Cu) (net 2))
 (segment (start 208.026 90.551) (end 208.026 91.694) (width 1) (layer F.Cu) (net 2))
 (segment (start 208.026 90.551) (end 208.026 94.869) (width 1) (layer F.Cu) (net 2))
 (segment (start 208.026 86.106) (end 208.026 90.551) (width 1) (layer F.Cu) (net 2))
 (segment (start 208.026 97.409) (end 208.026 94.869) (width 1) (layer F.Cu) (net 2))
 (segment (start 216.535 104.775) (end 210.82 104.775) (width 1) (layer F.Cu) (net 2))
 (segment (start 208.026 101.981) (end 208.026 97.409) (width 1) (layer F.Cu) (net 2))
 (segment (start 217.805 106.045) (end 216.535 104.775) (width 1) (layer B.Cu) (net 2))
 (segment (start 219.71 106.045) (end 217.805 106.045) (width 1) (layer B.Cu) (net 2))
 (segment (start 205.105 83.185) (end 201.295 79.375) (width 1) (layer B.Cu) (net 2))
 (segment (start 205.105 83.185) (end 208.026 86.106) (width 1) (layer F.Cu) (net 2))
 (segment (start 208.28 104.14) (end 209.2325 103.1875) (width 1) (layer F.Cu) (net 2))
 (segment (start 203.835 104.14) (end 208.28 104.14) (width 1) (layer F.Cu) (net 2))
 (segment (start 210.82 104.775) (end 209.2325 103.1875) (width 1) (layer F.Cu) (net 2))
 (segment (start 209.2325 103.1875) (end 208.026 101.981) (width 1) (layer F.Cu) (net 2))
 (segment (start 195.58 94.996) (end 199.39 94.996) (width 1) (layer B.Cu) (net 2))
 (segment (start 199.39 94.996) (end 201.295 94.996) (width 1) (layer B.Cu) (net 2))
 (segment (start 207.899 94.996) (end 208.026 94.869) (width 1) (layer F.Cu) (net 2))
 (segment (start 201.295 94.996) (end 207.899 94.996) (width 1) (layer F.Cu) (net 2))
 (segment (start 201.041 79.121) (end 201.295 79.375) (width 1) (layer B.Cu) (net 2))
 (segment (start 199.39 79.121) (end 201.041 79.121) (width 1) (layer B.Cu) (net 2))
 (segment (start 226.314 94.488) (end 226.314 91.948) (width 1) (layer B.Cu) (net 1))
 (segment (start 226.314 91.948) (end 226.314 89.916) (width 1) (layer B.Cu) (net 1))
 (segment (start 222.32 85.922) (end 214.884 85.922) (width 1) (layer B.Cu) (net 1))
 (segment (start 226.314 89.916) (end 222.32 85.922) (width 1) (layer B.Cu) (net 1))
 (segment (start 213.995 95.4278) (end 213.995 93.98) (width 0.5) (layer F.Cu) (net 6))
 (segment (start 213.995 93.98) (end 214.63 93.345) (width 0.5) (layer F.Cu) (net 6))
 (segment (start 214.63 93.345) (end 216.535 93.345) (width 0.5) (layer F.Cu) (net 6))
 (segment (start 221.615 92.326002) (end 221.615 91.82) (width 0.5) (layer F.Cu) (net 6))
 (segment (start 219.651001 94.290001) (end 221.615 92.326002) (width 0.5) (layer F.Cu) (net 6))
 (segment (start 217.480001 94.290001) (end 219.651001 94.290001) (width 0.5) (layer F.Cu) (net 6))
 (segment (start 216.535 93.345) (end 217.480001 94.290001) (width 0.5) (layer F.Cu) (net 6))
 (segment (start 221.615 91.82) (end 221.615 91.313998) (width 0.5) (layer F.Cu) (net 6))
 (segment (start 223.646 94.36) (end 223.774 94.488) (width 1) (layer B.Cu) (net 4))
 (segment (start 221.615 94.36) (end 223.646 94.36) (width 1) (layer B.Cu) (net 4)))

